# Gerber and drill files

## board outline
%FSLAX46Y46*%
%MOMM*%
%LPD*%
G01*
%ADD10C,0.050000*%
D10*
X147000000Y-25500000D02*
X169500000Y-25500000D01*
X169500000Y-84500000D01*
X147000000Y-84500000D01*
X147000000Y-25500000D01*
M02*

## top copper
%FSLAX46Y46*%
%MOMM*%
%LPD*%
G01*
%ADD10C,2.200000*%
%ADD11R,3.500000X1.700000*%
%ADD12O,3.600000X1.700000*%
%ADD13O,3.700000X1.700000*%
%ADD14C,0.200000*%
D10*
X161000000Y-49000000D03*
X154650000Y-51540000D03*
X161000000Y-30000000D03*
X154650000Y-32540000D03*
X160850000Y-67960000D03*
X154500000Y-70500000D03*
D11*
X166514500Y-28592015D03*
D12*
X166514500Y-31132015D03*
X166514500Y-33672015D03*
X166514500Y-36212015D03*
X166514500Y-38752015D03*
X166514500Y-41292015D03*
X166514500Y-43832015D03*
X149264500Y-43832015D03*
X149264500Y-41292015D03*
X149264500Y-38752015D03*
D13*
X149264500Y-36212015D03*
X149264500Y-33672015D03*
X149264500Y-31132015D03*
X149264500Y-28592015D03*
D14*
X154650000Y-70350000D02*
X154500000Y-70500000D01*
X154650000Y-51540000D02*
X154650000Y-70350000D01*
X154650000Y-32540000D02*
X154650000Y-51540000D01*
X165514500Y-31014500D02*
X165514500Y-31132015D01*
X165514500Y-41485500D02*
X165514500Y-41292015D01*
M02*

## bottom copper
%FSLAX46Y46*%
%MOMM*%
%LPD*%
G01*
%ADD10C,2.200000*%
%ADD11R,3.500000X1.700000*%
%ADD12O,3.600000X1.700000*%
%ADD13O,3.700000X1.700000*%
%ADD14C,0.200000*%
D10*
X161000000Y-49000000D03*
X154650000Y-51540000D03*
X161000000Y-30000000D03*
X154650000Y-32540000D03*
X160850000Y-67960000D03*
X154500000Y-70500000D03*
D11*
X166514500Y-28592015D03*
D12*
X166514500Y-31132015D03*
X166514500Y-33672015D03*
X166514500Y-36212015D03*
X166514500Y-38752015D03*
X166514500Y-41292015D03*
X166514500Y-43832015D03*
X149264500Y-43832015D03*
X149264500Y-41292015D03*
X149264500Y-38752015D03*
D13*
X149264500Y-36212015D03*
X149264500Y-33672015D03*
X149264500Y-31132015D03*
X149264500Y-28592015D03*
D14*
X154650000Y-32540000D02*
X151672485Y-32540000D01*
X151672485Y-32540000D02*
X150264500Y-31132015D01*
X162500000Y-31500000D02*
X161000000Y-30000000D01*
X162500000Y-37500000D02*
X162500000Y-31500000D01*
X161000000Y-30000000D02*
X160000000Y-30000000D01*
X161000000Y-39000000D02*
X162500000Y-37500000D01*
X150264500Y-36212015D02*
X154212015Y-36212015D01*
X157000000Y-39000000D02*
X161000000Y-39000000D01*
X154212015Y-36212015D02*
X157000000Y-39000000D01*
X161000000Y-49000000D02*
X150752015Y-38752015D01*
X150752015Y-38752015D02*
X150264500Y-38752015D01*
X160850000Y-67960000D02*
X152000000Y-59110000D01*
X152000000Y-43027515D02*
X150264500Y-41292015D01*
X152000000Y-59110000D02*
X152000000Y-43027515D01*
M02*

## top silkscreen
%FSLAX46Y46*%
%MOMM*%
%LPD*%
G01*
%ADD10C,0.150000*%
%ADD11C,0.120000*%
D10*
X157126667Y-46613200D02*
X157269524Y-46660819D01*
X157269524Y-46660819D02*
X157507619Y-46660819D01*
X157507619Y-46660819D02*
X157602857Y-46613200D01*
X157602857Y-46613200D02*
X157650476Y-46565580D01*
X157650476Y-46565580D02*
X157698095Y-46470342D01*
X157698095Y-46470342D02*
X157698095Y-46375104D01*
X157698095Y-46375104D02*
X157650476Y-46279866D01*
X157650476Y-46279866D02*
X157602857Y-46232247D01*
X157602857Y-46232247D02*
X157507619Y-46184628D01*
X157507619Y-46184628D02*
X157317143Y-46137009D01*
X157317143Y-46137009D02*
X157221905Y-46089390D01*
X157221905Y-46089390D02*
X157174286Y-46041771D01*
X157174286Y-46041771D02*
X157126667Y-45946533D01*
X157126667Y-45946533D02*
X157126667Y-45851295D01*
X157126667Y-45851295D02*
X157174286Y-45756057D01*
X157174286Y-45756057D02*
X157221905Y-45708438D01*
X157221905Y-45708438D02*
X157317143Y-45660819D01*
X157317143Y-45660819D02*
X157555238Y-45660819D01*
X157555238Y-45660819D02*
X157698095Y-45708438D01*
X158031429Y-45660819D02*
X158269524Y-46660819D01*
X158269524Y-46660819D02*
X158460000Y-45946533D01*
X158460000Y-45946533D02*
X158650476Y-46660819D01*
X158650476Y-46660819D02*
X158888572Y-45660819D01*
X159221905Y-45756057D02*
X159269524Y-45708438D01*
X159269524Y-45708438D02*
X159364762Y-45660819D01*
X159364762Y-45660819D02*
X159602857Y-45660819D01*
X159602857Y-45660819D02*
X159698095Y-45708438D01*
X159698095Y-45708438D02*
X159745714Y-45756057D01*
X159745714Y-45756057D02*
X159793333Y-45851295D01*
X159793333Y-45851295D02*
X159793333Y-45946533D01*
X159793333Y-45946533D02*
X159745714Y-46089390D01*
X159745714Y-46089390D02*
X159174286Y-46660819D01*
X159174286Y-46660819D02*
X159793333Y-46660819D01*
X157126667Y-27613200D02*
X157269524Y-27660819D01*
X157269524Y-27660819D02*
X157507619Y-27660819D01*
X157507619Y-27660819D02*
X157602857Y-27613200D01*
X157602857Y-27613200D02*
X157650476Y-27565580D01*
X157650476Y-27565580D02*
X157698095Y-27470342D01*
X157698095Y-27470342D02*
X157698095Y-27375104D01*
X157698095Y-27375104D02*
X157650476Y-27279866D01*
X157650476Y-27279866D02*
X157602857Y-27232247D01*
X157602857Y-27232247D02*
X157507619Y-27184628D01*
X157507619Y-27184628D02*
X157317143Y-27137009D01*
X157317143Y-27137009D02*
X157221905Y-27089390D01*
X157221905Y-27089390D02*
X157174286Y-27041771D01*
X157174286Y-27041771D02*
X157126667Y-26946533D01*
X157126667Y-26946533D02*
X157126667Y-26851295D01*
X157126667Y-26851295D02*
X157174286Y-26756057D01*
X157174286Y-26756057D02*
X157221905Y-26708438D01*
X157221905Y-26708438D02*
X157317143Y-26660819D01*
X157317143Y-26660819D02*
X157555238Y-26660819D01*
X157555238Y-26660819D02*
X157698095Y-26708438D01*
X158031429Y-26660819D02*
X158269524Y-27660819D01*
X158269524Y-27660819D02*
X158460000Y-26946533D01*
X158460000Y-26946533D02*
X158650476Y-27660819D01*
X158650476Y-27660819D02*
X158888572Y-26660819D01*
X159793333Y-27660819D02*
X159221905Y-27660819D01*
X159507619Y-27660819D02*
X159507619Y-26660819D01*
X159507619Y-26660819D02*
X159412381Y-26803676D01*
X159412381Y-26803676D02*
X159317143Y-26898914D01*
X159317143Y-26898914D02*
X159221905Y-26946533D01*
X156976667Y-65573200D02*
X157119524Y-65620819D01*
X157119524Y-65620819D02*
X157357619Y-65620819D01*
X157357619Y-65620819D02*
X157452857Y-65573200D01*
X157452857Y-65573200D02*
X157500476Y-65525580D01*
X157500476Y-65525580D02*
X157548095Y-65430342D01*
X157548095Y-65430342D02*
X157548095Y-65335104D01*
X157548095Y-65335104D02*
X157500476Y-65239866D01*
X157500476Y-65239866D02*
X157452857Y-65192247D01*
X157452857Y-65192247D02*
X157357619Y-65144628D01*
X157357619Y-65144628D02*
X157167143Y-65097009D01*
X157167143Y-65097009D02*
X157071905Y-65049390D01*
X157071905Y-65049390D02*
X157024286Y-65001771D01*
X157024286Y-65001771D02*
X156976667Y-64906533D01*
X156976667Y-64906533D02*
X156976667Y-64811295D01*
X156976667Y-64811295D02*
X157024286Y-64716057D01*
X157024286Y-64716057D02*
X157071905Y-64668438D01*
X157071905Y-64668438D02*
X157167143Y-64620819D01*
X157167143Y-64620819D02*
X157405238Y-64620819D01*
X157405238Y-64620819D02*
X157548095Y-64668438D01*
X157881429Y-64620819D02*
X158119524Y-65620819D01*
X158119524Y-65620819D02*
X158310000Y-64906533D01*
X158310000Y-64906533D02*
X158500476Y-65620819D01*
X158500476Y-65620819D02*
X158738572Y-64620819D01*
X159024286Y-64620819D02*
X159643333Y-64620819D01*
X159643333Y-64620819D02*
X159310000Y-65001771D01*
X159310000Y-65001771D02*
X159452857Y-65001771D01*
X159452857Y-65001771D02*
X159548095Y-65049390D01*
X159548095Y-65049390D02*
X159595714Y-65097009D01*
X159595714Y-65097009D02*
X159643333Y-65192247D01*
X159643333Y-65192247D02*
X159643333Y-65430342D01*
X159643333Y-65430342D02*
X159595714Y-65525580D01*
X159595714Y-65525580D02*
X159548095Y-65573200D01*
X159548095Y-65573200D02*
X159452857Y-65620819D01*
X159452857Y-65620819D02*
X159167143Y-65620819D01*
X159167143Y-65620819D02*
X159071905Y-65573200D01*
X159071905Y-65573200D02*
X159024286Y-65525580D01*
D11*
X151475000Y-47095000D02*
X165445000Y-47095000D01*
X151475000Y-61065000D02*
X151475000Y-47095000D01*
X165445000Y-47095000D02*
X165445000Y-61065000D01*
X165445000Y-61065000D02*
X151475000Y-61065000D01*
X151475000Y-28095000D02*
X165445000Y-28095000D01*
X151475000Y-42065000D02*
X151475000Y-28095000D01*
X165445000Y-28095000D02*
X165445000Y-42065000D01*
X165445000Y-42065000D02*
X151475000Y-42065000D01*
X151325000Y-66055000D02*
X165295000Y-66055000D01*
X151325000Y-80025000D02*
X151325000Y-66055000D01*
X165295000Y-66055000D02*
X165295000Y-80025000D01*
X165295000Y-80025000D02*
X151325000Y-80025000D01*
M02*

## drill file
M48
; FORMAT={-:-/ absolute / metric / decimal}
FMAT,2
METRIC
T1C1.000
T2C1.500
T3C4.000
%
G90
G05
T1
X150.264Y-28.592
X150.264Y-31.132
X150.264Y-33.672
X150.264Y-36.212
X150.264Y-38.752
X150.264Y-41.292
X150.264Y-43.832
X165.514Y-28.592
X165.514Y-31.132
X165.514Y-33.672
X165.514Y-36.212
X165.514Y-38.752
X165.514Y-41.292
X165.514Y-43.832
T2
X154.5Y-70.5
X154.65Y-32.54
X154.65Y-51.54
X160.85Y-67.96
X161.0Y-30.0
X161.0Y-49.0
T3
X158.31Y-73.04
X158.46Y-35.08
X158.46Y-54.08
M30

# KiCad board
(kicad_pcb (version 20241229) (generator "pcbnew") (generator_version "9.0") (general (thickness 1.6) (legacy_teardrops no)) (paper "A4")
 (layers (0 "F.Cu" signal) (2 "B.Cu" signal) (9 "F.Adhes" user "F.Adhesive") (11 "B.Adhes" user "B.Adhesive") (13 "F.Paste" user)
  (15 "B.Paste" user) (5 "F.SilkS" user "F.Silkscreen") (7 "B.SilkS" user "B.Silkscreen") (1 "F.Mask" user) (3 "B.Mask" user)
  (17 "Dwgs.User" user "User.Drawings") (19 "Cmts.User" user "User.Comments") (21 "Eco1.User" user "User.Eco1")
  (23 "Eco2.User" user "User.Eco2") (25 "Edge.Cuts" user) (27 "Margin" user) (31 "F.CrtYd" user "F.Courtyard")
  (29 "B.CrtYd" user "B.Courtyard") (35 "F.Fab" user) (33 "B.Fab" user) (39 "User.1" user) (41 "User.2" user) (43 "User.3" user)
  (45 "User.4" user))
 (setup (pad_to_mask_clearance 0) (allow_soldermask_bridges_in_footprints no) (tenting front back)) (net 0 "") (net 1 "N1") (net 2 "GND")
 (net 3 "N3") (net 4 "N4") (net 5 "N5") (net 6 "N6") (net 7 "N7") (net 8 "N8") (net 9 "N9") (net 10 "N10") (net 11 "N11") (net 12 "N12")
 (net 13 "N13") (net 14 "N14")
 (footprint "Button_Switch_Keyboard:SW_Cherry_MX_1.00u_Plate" (layer "F.Cu") (at 161 49)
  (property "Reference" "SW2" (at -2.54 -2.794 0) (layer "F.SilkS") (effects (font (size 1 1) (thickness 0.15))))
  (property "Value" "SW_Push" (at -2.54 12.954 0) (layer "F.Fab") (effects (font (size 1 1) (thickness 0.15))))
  (fp_line (start -9.525 -1.905) (end 4.445 -1.905) (stroke (width 0.12) (type solid)) (layer "F.SilkS"))
  (fp_line (start -9.525 12.065) (end -9.525 -1.905) (stroke (width 0.12) (type solid)) (layer "F.SilkS"))
  (fp_line (start 4.445 -1.905) (end 4.445 12.065) (stroke (width 0.12) (type solid)) (layer "F.SilkS"))
  (fp_line (start 4.445 12.065) (end -9.525 12.065) (stroke (width 0.12) (type solid)) (layer "F.SilkS"))
  (pad "" np_thru_hole circle (at -2.54 5.08) (size 4 4) (drill 4) (layers "*.Cu" "*.Mask"))
  (pad "1" thru_hole circle (at 0 0) (size 2.2 2.2) (drill 1.5) (layers "*.Cu" "*.Mask") (remove_unused_layers no) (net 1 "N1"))
  (pad "2" thru_hole circle (at -6.35 2.54) (size 2.2 2.2) (drill 1.5) (layers "*.Cu" "*.Mask") (remove_unused_layers no) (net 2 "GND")))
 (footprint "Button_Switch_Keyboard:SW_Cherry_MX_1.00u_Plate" (layer "F.Cu") (at 161 30)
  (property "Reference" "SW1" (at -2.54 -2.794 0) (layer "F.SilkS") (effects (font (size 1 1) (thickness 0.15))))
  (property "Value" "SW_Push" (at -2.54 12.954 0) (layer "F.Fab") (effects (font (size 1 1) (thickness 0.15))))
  (fp_line (start -9.525 -1.905) (end 4.445 -1.905) (stroke (width 0.12) (type solid)) (layer "F.SilkS"))
  (fp_line (start -9.525 12.065) (end -9.525 -1.905) (stroke (width 0.12) (type solid)) (layer "F.SilkS"))
  (fp_line (start 4.445 -1.905) (end 4.445 12.065) (stroke (width 0.12) (type solid)) (layer "F.SilkS"))
  (fp_line (start 4.445 12.065) (end -9.525 12.065) (stroke (width 0.12) (type solid)) (layer "F.SilkS"))
  (pad "" np_thru_hole circle (at -2.54 5.08) (size 4 4) (drill 4) (layers "*.Cu" "*.Mask"))
  (pad "1" thru_hole circle (at 0 0) (size 2.2 2.2) (drill 1.5) (layers "*.Cu" "*.Mask") (remove_unused_layers no) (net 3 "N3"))
  (pad "2" thru_hole circle (at -6.35 2.54) (size 2.2 2.2) (drill 1.5) (layers "*.Cu" "*.Mask") (remove_unused_layers no) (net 2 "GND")))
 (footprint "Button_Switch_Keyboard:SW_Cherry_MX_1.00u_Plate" (layer "F.Cu") (at 160.85 67.96)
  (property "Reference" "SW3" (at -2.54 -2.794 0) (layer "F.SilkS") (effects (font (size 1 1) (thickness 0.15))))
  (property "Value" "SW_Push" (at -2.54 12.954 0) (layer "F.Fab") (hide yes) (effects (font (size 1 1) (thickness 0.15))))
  (fp_line (start -9.525 -1.905) (end 4.445 -1.905) (stroke (width 0.12) (type solid)) (layer "F.SilkS"))
  (fp_line (start -9.525 12.065) (end -9.525 -1.905) (stroke (width 0.12) (type solid)) (layer "F.SilkS"))
  (fp_line (start 4.445 -1.905) (end 4.445 12.065) (stroke (width 0.12) (type solid)) (layer "F.SilkS"))
  (fp_line (start 4.445 12.065) (end -9.525 12.065) (stroke (width 0.12) (type solid)) (layer "F.SilkS"))
  (pad "" np_thru_hole circle (at -2.54 5.08) (size 4 4) (drill 4) (layers "*.Cu" "*.Mask"))
  (pad "1" thru_hole circle (at 0 0) (size 2.2 2.2) (drill 1.5) (layers "*.Cu" "*.Mask") (remove_unused_layers no) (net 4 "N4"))
  (pad "2" thru_hole circle (at -6.35 2.54) (size 2.2 2.2) (drill 1.5) (layers "*.Cu" "*.Mask") (remove_unused_layers no) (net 2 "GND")))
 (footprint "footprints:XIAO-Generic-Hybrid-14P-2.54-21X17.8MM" (layer "B.Cu") (at 157.8895 36.212015 180)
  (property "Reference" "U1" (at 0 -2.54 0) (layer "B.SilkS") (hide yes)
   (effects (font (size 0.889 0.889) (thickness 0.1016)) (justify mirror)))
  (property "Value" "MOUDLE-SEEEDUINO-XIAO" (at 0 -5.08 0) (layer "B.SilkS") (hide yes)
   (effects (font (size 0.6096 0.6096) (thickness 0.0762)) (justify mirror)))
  (pad "1" thru_hole rect (at -7.625 7.62 180) (size 3.5 1.7) (drill 1 (offset -1 0)) (layers "*.Cu" "*.Mask") (remove_unused_layers no)
   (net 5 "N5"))
  (pad "2" thru_hole oval (at -7.625 5.08 180) (size 3.6 1.7) (drill 1 (offset -1 0)) (layers "*.Cu" "*.Mask") (remove_unused_layers no)
   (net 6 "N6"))
  (pad "3" thru_hole oval (at -7.625 2.54 180) (size 3.6 1.7) (drill 1 (offset -1 0)) (layers "*.Cu" "*.Mask") (remove_unused_layers no)
   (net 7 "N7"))
  (pad "4" thru_hole oval (at -7.625 0 180) (size 3.6 1.7) (drill 1 (offset -1 0)) (layers "*.Cu" "*.Mask") (remove_unused_layers no)
   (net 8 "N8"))
  (pad "5" thru_hole oval (at -7.625 -2.54 180) (size 3.6 1.7) (drill 1 (offset -1 0)) (layers "*.Cu" "*.Mask") (remove_unused_layers no)
   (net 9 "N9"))
  (pad "6" thru_hole oval (at -7.625 -5.08) (size 3.6 1.7) (drill 1 (offset 1 0)) (layers "*.Cu" "*.Mask") (remove_unused_layers no)
   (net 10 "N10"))
  (pad "7" thru_hole oval (at -7.625 -7.62 180) (size 3.6 1.7) (drill 1 (offset -1 0)) (layers "*.Cu" "*.Mask") (remove_unused_layers no)
   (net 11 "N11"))
  (pad "8" thru_hole oval (at 7.625 -7.62 180) (size 3.6 1.7) (drill 1 (offset 1 0)) (layers "*.Cu" "*.Mask") (remove_unused_layers no)
   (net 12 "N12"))
  (pad "9" thru_hole oval (at 7.625 -5.08 180) (size 3.6 1.7) (drill 1 (offset 1 0)) (layers "*.Cu" "*.Mask") (remove_unused_layers no)
   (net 4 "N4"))
  (pad "10" thru_hole oval (at 7.625 -2.54 180) (size 3.6 1.7) (drill 1 (offset 1 0)) (layers "*.Cu" "*.Mask") (remove_unused_layers no)
   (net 1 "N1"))
  (pad "11" thru_hole oval (at 7.625 0 180) (size 3.7 1.7) (drill 1 (offset 1 0)) (layers "*.Cu" "*.Mask") (remove_unused_layers no)
   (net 3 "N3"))
  (pad "12" thru_hole oval (at 7.625 2.54 180) (size 3.7 1.7) (drill 1 (offset 1 0)) (layers "*.Cu" "*.Mask") (remove_unused_layers no)
   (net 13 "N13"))
  (pad "13" thru_hole oval (at 7.625 5.08 180) (size 3.7 1.7) (drill 1 (offset 1 0)) (layers "*.Cu" "*.Mask") (remove_unused_layers no)
   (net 2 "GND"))
  (pad "14" thru_hole oval (at 7.625 7.62 180) (size 3.7 1.7) (drill 1 (offset 1 0)) (layers "*.Cu" "*.Mask") (remove_unused_layers no)
   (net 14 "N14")))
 (gr_rect (start 147 25.5) (end 169.5 84.5) (stroke (width 0.05) (type default)) (fill no) (layer "Edge.Cuts"))
 (segment (start 154.65 70.35) (end 154.5 70.5) (width 0.2) (layer "F.Cu") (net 2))
 (segment (start 154.65 51.54) (end 154.65 70.35) (width 0.2) (layer "F.Cu") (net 2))
 (segment (start 154.65 32.54) (end 154.65 51.54) (width 0.2) (layer "F.Cu") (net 2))
 (segment (start 154.65 32.54) (end 151.672485 32.54) (width 0.2) (layer "B.Cu") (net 2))
 (segment (start 151.672485 32.54) (end 150.2645 31.132015) (width 0.2) (layer "B.Cu") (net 2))
 (segment (start 162.5 31.5) (end 161 30) (width 0.2) (layer "B.Cu") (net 3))
 (segment (start 162.5 37.5) (end 162.5 31.5) (width 0.2) (layer "B.Cu") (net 3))
 (segment (start 161 30) (end 160 30) (width 0.2) (layer "B.Cu") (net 3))
 (segment (start 161 39) (end 162.5 37.5) (width 0.2) (layer "B.Cu") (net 3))
 (segment (start 150.2645 36.212015) (end 154.212015 36.212015) (width 0.2) (layer "B.Cu") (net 3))
 (segment (start 157 39) (end 161 39) (width 0.2) (layer "B.Cu") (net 3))
 (segment (start 154.212015 36.212015) (end 157 39) (width 0.2) (layer "B.Cu") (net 3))
 (segment (start 161 49) (end 150.752015 38.752015) (width 0.2) (layer "B.Cu") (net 1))
 (segment (start 150.752015 38.752015) (end 150.2645 38.752015) (width 0.2) (layer "B.Cu") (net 1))
 (segment (start 160.85 67.96) (end 152 59.11) (width 0.2) (layer "B.Cu") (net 4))
 (segment (start 152 43.027515) (end 150.2645 41.292015) (width 0.2) (layer "B.Cu") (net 4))
 (segment (start 152 59.11) (end 152 43.027515) (width 0.2) (layer "B.Cu") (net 4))
 (segment (start 165.5145 31.0145) (end 165.5145 31.132015) (width 0.2) (layer "F.Cu") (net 6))
 (segment (start 165.5145 41.4855) (end 165.5145 41.292015) (width 0.2) (layer "F.Cu") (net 10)))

